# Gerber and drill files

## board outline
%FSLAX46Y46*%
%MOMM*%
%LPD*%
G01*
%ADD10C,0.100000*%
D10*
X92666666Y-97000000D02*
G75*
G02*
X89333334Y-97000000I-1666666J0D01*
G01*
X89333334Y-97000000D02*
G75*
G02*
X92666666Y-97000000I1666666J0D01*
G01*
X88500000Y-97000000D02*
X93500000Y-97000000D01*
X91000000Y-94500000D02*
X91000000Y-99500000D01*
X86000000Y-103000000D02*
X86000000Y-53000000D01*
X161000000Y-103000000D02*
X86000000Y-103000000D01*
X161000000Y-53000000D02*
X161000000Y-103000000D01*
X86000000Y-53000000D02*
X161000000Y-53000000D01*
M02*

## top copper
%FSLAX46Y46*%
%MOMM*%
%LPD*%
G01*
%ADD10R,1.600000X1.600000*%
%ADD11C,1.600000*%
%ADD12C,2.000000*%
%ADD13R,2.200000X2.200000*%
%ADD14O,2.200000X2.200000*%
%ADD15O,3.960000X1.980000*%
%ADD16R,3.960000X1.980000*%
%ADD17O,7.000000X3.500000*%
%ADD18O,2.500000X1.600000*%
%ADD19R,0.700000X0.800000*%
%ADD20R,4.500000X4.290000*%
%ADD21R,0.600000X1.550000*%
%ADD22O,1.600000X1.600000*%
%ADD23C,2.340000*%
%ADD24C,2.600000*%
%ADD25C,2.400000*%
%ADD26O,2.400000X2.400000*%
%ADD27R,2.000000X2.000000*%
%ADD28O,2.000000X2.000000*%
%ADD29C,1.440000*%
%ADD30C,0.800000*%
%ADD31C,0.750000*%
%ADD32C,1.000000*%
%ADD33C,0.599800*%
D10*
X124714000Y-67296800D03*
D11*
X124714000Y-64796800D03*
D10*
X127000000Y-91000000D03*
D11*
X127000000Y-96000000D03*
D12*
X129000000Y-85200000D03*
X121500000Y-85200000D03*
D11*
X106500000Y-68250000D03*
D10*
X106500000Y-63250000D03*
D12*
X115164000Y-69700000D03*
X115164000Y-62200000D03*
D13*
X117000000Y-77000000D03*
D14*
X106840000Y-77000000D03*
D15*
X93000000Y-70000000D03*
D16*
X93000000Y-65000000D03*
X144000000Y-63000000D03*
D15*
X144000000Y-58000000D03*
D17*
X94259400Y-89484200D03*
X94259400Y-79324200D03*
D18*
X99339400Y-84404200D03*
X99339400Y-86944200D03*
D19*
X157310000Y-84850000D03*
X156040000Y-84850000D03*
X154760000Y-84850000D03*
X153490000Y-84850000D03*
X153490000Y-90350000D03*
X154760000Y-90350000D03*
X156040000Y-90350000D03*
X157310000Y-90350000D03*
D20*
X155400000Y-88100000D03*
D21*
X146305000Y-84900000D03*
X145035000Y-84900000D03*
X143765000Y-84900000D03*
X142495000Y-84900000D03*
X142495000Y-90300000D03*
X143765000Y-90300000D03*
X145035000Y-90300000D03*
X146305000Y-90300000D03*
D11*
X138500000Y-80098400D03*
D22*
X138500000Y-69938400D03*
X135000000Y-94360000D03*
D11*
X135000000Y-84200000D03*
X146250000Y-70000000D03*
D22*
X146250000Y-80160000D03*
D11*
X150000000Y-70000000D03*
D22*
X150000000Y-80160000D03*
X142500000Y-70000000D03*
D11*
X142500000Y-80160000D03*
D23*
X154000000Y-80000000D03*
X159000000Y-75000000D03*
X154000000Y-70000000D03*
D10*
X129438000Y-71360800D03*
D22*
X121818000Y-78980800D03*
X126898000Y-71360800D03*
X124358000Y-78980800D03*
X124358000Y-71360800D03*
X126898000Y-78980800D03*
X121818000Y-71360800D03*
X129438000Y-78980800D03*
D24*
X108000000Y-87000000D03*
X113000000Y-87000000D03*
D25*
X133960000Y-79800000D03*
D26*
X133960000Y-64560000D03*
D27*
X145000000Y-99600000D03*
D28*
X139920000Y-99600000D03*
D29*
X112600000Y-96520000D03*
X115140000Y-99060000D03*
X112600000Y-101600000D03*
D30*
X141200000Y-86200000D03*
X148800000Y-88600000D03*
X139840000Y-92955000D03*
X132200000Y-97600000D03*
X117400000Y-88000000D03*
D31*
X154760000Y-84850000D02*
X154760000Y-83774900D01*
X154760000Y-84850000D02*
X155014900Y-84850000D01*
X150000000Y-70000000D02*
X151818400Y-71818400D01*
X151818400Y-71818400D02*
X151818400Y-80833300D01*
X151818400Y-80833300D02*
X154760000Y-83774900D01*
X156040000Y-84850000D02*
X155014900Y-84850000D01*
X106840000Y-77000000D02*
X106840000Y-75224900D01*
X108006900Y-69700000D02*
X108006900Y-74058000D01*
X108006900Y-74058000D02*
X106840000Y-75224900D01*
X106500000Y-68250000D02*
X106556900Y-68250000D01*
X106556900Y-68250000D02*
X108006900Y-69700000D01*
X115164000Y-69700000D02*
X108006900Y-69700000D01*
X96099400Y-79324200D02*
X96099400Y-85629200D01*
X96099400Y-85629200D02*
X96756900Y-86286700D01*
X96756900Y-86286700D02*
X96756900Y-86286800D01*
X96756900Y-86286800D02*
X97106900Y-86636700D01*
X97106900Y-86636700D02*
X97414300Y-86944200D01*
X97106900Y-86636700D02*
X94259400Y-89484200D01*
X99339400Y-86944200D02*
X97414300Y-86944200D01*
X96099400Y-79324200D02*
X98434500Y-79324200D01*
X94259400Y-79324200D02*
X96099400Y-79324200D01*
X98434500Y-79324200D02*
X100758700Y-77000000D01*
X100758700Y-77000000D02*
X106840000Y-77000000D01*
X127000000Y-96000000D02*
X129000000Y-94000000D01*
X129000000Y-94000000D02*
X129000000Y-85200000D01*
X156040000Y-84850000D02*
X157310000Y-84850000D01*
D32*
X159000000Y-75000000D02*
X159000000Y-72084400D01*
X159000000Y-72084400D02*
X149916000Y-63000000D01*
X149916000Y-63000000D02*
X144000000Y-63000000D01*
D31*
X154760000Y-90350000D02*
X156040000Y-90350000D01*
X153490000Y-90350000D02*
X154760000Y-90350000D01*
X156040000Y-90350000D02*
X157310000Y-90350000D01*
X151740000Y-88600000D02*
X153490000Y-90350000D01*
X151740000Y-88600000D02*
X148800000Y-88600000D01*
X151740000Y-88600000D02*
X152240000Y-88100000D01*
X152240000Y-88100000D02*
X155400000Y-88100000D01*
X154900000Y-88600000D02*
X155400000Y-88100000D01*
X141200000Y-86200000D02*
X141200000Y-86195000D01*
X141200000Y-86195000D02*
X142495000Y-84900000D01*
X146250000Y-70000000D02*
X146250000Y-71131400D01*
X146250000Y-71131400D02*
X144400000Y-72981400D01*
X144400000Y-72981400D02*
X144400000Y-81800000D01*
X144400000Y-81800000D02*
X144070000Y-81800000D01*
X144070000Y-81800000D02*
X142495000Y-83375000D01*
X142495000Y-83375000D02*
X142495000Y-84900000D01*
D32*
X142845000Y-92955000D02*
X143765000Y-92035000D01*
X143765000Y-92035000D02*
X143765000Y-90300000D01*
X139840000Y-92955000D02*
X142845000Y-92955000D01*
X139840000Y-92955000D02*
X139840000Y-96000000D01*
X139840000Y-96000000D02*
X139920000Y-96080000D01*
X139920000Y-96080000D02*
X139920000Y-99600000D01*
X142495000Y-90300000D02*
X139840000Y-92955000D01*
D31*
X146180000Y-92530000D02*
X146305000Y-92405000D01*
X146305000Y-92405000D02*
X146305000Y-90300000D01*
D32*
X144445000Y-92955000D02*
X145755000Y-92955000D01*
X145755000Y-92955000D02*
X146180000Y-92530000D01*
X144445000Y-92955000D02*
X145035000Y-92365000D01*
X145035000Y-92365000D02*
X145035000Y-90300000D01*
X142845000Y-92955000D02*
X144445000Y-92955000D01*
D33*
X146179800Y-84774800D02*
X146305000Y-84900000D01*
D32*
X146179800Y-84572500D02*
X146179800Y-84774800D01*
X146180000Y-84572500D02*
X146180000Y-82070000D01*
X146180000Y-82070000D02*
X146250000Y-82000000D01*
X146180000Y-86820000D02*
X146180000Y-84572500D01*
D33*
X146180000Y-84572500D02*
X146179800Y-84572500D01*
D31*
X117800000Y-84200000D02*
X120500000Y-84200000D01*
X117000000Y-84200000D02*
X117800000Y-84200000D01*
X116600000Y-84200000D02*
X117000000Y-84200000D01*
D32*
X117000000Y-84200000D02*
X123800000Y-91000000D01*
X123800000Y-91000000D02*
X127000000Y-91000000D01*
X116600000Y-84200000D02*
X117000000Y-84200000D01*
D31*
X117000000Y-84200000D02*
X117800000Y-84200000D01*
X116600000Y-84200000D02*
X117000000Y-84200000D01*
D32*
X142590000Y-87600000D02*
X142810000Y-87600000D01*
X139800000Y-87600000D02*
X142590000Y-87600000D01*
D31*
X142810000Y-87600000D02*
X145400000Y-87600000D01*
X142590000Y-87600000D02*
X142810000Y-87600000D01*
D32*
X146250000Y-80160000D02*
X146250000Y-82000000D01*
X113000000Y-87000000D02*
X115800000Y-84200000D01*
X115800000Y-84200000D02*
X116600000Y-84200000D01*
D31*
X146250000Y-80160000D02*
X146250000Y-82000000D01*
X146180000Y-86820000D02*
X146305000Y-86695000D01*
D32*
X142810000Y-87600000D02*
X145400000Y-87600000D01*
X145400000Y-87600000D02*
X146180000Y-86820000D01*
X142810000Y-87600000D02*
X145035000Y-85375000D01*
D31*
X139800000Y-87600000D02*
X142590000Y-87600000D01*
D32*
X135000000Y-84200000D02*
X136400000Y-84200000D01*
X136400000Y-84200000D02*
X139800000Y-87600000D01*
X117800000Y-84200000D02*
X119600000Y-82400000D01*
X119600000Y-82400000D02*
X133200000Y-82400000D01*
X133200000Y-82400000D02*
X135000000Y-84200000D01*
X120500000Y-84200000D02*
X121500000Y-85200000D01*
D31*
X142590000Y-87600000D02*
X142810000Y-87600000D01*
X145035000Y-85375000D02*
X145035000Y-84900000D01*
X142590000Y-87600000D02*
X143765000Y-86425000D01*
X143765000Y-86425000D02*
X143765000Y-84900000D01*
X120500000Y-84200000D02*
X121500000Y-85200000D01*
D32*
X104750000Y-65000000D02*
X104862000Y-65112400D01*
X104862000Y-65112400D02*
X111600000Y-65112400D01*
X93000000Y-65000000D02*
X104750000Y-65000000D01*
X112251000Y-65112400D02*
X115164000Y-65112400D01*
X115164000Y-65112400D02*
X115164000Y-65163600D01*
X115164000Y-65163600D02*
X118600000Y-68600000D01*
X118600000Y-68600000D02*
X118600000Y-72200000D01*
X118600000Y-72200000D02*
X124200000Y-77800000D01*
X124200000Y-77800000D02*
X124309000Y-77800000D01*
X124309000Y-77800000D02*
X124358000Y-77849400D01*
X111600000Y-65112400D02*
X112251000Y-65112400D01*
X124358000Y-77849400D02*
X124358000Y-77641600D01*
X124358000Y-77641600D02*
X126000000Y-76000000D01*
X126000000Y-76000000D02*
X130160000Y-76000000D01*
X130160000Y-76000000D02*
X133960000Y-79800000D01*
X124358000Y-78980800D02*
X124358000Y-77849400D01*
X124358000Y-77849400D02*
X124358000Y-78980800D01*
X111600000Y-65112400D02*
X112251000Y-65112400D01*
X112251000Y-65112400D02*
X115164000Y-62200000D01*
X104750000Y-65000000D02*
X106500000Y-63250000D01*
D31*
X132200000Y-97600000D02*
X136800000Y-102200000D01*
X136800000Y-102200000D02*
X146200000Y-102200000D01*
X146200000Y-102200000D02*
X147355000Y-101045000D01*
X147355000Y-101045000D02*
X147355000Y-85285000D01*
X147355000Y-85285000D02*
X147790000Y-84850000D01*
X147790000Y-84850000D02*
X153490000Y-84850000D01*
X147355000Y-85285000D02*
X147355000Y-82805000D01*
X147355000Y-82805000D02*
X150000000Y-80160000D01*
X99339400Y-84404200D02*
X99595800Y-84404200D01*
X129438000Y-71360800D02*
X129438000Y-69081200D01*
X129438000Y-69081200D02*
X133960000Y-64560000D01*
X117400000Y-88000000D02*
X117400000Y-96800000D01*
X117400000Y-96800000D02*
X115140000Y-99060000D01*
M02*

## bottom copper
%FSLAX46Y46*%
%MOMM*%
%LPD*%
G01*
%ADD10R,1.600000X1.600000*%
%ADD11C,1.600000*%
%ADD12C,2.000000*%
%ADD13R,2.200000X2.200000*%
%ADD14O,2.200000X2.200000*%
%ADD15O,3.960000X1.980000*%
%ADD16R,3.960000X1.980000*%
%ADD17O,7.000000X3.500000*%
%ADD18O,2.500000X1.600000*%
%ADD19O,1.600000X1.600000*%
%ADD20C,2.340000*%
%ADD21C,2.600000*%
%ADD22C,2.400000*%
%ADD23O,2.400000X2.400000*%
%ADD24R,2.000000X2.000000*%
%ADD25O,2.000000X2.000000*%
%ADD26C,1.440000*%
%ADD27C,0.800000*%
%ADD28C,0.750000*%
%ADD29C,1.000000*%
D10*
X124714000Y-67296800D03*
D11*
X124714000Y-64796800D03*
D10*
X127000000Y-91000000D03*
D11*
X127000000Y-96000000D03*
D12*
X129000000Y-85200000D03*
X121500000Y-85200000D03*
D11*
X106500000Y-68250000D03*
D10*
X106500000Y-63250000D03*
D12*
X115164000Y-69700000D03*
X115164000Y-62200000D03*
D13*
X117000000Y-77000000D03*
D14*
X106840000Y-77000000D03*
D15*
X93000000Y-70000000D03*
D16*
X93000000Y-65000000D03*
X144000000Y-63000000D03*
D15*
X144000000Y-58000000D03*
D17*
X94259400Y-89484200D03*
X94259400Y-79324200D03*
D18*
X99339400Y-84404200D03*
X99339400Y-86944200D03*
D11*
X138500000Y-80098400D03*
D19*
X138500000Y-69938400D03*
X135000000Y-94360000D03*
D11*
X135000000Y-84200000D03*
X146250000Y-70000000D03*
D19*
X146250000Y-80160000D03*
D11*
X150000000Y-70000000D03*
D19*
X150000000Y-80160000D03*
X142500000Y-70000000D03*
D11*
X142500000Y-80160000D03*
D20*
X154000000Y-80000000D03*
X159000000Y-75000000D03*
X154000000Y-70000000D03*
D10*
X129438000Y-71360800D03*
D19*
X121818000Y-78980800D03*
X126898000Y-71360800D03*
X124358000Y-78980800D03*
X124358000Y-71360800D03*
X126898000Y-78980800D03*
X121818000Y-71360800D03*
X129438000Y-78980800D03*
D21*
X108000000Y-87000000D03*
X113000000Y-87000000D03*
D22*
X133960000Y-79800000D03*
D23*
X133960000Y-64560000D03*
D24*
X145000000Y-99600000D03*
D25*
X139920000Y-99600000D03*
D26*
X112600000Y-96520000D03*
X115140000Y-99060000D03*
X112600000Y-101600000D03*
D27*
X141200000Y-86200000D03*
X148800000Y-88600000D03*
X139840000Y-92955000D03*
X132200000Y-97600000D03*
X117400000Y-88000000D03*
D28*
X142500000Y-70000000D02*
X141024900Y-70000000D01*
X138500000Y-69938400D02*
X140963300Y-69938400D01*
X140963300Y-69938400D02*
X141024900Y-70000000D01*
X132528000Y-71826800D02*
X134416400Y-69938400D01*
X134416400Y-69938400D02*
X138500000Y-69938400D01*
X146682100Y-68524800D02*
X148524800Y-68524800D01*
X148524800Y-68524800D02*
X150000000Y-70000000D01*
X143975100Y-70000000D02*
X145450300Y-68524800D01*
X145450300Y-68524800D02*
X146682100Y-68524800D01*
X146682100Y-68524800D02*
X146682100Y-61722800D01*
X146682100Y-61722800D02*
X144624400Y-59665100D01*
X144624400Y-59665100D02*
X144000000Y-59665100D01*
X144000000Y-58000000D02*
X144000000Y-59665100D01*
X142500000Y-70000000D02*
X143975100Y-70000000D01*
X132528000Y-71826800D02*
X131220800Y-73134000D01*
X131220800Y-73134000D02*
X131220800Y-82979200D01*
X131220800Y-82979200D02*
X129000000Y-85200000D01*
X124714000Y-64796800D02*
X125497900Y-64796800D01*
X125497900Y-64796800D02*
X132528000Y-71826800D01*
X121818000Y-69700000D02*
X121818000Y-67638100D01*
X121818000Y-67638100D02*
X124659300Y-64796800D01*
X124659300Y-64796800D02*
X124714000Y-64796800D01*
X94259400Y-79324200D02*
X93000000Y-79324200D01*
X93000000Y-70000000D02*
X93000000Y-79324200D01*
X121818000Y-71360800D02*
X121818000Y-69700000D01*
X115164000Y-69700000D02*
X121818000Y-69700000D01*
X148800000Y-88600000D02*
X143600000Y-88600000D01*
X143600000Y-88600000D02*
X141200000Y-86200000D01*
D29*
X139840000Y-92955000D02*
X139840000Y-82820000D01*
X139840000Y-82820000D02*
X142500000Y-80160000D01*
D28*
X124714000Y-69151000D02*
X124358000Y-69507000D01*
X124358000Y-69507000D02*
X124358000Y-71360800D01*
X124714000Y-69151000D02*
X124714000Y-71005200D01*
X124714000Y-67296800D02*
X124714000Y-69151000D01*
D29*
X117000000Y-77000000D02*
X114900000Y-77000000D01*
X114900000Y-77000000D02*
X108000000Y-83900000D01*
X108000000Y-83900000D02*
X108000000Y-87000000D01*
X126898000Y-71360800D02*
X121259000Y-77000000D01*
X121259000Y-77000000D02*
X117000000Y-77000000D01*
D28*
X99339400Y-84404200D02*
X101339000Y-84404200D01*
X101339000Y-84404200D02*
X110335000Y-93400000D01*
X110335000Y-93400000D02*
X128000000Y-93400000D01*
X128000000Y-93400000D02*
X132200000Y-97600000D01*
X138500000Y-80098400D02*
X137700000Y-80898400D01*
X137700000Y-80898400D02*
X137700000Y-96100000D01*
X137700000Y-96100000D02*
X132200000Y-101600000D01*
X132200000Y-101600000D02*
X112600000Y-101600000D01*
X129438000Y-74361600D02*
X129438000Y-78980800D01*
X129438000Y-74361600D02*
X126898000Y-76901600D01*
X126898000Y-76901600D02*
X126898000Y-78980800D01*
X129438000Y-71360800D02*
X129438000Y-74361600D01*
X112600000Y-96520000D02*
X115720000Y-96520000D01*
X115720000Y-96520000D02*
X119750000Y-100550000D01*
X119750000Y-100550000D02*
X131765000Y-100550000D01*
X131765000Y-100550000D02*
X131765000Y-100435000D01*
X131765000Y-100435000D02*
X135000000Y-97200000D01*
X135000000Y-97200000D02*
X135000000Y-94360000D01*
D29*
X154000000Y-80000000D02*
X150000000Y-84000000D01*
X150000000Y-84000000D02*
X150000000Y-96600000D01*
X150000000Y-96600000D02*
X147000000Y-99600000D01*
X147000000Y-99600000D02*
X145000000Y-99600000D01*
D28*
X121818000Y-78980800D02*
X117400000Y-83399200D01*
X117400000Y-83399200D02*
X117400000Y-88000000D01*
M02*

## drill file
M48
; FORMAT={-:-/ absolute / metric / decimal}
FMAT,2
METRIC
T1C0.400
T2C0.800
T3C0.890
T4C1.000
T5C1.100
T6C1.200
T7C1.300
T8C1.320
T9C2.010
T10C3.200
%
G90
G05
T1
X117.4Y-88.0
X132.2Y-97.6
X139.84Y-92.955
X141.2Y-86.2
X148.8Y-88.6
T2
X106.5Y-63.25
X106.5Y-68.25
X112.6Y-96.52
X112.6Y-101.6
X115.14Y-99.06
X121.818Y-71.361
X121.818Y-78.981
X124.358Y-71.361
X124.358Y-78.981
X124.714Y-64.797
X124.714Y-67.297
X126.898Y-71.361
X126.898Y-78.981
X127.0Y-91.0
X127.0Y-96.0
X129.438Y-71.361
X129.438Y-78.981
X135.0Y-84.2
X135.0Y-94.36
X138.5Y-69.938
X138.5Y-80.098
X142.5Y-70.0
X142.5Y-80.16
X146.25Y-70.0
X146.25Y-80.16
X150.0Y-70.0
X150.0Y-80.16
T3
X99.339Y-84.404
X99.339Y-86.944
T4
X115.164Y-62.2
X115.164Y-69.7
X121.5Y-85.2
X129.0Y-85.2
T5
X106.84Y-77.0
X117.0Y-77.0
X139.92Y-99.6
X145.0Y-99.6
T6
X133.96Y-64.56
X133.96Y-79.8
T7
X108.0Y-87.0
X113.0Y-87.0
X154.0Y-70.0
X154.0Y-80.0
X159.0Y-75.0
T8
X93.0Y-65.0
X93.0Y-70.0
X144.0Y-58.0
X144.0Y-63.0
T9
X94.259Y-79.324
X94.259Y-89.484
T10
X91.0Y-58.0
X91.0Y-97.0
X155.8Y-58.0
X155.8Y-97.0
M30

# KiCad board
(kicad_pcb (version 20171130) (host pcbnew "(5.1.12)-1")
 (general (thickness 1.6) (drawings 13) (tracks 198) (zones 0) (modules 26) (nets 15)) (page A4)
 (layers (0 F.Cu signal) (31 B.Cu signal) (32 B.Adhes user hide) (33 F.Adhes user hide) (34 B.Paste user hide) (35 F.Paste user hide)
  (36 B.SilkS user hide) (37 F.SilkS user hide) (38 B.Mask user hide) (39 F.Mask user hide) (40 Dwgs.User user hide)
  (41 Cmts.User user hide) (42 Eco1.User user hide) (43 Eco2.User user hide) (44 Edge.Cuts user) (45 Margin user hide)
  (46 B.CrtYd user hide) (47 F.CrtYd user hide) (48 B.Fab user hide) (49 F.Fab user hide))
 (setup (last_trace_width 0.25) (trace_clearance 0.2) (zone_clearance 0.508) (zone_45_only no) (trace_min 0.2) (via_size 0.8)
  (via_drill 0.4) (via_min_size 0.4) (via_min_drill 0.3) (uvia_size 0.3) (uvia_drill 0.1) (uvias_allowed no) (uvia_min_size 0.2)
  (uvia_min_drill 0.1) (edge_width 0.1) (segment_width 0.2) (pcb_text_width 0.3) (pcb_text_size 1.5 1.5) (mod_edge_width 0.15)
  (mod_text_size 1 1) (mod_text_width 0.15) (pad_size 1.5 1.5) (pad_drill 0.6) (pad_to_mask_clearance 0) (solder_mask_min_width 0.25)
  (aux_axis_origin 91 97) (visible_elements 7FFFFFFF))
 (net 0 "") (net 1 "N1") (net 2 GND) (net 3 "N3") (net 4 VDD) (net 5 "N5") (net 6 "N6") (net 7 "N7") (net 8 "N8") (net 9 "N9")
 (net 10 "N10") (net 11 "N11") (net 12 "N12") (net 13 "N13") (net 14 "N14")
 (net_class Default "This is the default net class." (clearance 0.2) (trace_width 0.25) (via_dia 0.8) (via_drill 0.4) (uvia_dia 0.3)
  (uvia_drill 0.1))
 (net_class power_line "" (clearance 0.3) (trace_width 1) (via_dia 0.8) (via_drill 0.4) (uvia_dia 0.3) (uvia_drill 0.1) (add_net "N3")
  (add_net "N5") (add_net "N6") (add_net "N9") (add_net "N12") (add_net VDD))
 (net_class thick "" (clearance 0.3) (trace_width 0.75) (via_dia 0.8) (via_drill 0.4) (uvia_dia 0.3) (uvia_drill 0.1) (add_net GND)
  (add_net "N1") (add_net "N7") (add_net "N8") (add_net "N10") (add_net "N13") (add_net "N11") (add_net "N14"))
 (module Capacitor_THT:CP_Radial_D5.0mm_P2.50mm (layer F.Cu) (at 124.714 67.2968 90)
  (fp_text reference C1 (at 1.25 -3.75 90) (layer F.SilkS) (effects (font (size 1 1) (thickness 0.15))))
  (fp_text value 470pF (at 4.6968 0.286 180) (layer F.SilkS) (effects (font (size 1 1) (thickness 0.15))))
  (pad 1 thru_hole rect (at 0 0 90) (size 1.6 1.6) (drill 0.8) (layers *.Cu *.Mask) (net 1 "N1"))
  (pad 2 thru_hole circle (at 2.5 0 90) (size 1.6 1.6) (drill 0.8) (layers *.Cu *.Mask) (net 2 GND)))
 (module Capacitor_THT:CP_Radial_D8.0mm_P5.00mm (layer F.Cu) (at 127 91 270)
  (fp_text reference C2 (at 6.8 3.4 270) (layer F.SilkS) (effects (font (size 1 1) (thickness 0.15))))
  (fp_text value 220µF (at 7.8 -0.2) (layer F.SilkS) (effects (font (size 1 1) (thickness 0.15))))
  (pad 1 thru_hole rect (at 0 0 270) (size 1.6 1.6) (drill 0.8) (layers *.Cu *.Mask) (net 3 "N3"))
  (pad 2 thru_hole circle (at 5 0 270) (size 1.6 1.6) (drill 0.8) (layers *.Cu *.Mask) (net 2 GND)))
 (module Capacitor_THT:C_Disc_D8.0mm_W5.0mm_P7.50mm (layer F.Cu) (at 129 85.2 180)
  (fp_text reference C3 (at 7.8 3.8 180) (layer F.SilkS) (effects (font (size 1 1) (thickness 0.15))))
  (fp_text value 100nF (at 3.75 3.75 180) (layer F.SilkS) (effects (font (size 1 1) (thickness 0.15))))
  (pad 1 thru_hole circle (at 0 0 180) (size 2 2) (drill 1) (layers *.Cu *.Mask) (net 2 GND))
  (pad 2 thru_hole circle (at 7.5 0 180) (size 2 2) (drill 1) (layers *.Cu *.Mask) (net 3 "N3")))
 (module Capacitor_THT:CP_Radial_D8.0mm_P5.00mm (layer F.Cu) (at 106.5 63.25 270)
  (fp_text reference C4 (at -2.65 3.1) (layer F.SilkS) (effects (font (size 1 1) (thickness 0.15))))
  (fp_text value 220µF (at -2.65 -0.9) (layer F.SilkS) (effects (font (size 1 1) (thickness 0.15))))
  (pad 2 thru_hole circle (at 5 0 270) (size 1.6 1.6) (drill 0.8) (layers *.Cu *.Mask) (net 2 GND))
  (pad 1 thru_hole rect (at 0 0 270) (size 1.6 1.6) (drill 0.8) (layers *.Cu *.Mask) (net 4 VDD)))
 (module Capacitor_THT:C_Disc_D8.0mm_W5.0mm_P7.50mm (layer F.Cu) (at 115.164 62.2 270)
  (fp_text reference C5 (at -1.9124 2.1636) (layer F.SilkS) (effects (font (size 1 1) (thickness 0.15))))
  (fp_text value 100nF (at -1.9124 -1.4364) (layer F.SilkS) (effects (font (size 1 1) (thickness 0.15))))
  (pad 2 thru_hole circle (at 7.5 0 270) (size 2 2) (drill 1) (layers *.Cu *.Mask) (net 2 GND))
  (pad 1 thru_hole circle (at 0 0 270) (size 2 2) (drill 1) (layers *.Cu *.Mask) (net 4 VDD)))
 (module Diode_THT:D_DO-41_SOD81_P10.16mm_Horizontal (layer F.Cu) (at 117 77 180)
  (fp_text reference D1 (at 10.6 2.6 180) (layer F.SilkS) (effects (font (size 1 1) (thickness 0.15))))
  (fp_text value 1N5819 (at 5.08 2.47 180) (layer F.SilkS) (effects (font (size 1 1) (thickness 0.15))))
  (pad 1 thru_hole rect (at 0 0 180) (size 2.2 2.2) (drill 1.1) (layers *.Cu *.Mask) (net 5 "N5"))
  (pad 2 thru_hole oval (at 10.16 0 180) (size 2.2 2.2) (drill 1.1) (layers *.Cu *.Mask) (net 2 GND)))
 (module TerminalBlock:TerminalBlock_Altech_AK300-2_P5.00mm (layer F.Cu) (at 93 65 270)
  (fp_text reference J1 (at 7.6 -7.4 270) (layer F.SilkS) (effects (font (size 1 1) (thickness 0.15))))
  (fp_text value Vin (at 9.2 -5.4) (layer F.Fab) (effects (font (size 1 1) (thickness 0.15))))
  (pad 2 thru_hole oval (at 5 0 270) (size 1.98 3.96) (drill 1.32) (layers *.Cu *.Mask) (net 2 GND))
  (pad 1 thru_hole rect (at 0 0 270) (size 1.98 3.96) (drill 1.32) (layers *.Cu *.Mask) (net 4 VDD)))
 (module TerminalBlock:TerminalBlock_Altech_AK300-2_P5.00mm (layer F.Cu) (at 144 63 90)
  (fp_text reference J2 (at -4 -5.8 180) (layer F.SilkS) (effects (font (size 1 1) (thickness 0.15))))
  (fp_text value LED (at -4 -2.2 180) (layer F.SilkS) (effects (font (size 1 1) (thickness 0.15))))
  (pad 1 thru_hole rect (at 0 0 90) (size 1.98 3.96) (drill 1.32) (layers *.Cu *.Mask) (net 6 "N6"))
  (pad 2 thru_hole oval (at 5 0 90) (size 1.98 3.96) (drill 1.32) (layers *.Cu *.Mask) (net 2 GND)))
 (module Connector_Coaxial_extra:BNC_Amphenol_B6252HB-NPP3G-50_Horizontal (layer F.Cu) (at 99.3394 84.4042 90)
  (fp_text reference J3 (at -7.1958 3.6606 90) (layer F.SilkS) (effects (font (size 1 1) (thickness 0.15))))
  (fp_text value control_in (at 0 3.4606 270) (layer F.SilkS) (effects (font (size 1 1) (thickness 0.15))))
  (pad 2 thru_hole oval (at -5.08 -5.08 90) (size 3.5 7) (drill 2.01) (layers *.Cu *.Mask) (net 2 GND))
  (pad 2 thru_hole oval (at 5.08 -5.08 90) (size 3.5 7) (drill 2.01) (layers *.Cu *.Mask) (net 2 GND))
  (pad 1 thru_hole oval (at 0 0 90) (size 1.6 2.5) (drill 0.89) (layers *.Cu *.Mask) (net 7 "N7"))
  (pad 2 thru_hole oval (at -2.54 0 90) (size 1.6 2.5) (drill 0.89) (layers *.Cu *.Mask) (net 2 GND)))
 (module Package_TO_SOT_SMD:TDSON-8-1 (layer F.Cu) (at 155.4 87.6 270)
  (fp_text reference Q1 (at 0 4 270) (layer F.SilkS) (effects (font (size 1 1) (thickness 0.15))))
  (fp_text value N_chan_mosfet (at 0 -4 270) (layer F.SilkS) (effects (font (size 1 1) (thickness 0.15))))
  (pad 1 smd rect (at -2.75 -1.91 180) (size 0.7 0.8) (layers F.Cu F.Paste F.Mask) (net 2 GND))
  (pad 2 smd rect (at -2.75 -0.64 180) (size 0.7 0.8) (layers F.Cu F.Paste F.Mask) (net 2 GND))
  (pad 3 smd rect (at -2.75 0.64 180) (size 0.7 0.8) (layers F.Cu F.Paste F.Mask) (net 2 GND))
  (pad 4 smd rect (at -2.75 1.91 180) (size 0.7 0.8) (layers F.Cu F.Paste F.Mask) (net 7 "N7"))
  (pad 5 smd rect (at 2.75 1.91 180) (size 0.7 0.8) (layers F.Cu F.Paste F.Mask) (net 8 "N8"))
  (pad 5 smd rect (at 2.75 0.64 180) (size 0.7 0.8) (layers F.Cu F.Paste F.Mask) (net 8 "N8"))
  (pad 5 smd rect (at 2.75 -0.64 180) (size 0.7 0.8) (layers F.Cu F.Paste F.Mask) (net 8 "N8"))
  (pad 5 smd rect (at 2.75 -1.91 180) (size 0.7 0.8) (layers F.Cu F.Paste F.Mask) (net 8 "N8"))
  (pad 5 smd rect (at 0.5 0 180) (size 4.5 4.29) (layers F.Cu F.Mask) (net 8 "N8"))
  (pad "" smd rect (at 1.25 -1.09 180) (size 1.55 1.6) (layers F.Paste))
  (pad "" smd rect (at 1.25 1.09 180) (size 1.55 1.6) (layers F.Paste))
  (pad "" smd rect (at -0.75 -1.09 180) (size 1.55 1.2) (layers F.Paste))
  (pad "" smd rect (at -0.75 1.09 180) (size 1.55 1.2) (layers F.Paste)))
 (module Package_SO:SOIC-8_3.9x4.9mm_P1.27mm (layer F.Cu) (at 144.4 87.6 270)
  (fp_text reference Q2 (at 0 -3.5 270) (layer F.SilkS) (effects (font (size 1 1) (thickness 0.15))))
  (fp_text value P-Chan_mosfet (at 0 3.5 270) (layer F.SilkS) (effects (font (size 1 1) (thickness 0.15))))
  (pad 1 smd rect (at -2.7 -1.905 270) (size 1.55 0.6) (layers F.Cu F.Paste F.Mask) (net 3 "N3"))
  (pad 2 smd rect (at -2.7 -0.635 270) (size 1.55 0.6) (layers F.Cu F.Paste F.Mask) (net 3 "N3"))
  (pad 3 smd rect (at -2.7 0.635 270) (size 1.55 0.6) (layers F.Cu F.Paste F.Mask) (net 3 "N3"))
  (pad 4 smd rect (at -2.7 1.905 270) (size 1.55 0.6) (layers F.Cu F.Paste F.Mask) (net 8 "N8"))
  (pad 5 smd rect (at 2.7 1.905 270) (size 1.55 0.6) (layers F.Cu F.Paste F.Mask) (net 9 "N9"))
  (pad 6 smd rect (at 2.7 0.635 270) (size 1.55 0.6) (layers F.Cu F.Paste F.Mask) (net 9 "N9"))
  (pad 7 smd rect (at 2.7 -0.635 270) (size 1.55 0.6) (layers F.Cu F.Paste F.Mask) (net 9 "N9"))
  (pad 8 smd rect (at 2.7 -1.905 270) (size 1.55 0.6) (layers F.Cu F.Paste F.Mask) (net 9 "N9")))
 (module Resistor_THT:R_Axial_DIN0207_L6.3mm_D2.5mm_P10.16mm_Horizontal (layer F.Cu) (at 138.5 80.0984 90)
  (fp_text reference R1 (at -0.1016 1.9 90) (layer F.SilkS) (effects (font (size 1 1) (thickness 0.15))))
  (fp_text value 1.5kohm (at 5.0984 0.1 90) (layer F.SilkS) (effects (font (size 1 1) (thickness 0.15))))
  (pad 1 thru_hole circle (at 0 0 90) (size 1.6 1.6) (drill 0.8) (layers *.Cu *.Mask) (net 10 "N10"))
  (pad 2 thru_hole oval (at 10.16 0 90) (size 1.6 1.6) (drill 0.8) (layers *.Cu *.Mask) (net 2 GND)))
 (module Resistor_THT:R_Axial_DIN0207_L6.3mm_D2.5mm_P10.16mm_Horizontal (layer F.Cu) (at 135 84.2 270)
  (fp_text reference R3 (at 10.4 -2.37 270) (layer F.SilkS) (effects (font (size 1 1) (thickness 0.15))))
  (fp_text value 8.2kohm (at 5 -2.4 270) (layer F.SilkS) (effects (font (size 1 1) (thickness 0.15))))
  (pad 2 thru_hole oval (at 10.16 0 270) (size 1.6 1.6) (drill 0.8) (layers *.Cu *.Mask) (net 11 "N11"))
  (pad 1 thru_hole circle (at 0 0 270) (size 1.6 1.6) (drill 0.8) (layers *.Cu *.Mask) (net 3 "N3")))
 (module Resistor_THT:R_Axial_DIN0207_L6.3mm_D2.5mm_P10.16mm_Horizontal (layer F.Cu) (at 146.25 70 270)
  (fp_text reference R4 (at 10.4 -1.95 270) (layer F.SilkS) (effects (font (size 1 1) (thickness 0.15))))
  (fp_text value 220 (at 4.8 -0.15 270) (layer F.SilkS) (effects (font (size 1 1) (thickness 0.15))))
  (pad 1 thru_hole circle (at 0 0 270) (size 1.6 1.6) (drill 0.8) (layers *.Cu *.Mask) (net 8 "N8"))
  (pad 2 thru_hole oval (at 10.16 0 270) (size 1.6 1.6) (drill 0.8) (layers *.Cu *.Mask) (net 3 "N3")))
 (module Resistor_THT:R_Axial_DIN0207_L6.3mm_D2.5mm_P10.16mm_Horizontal (layer F.Cu) (at 150 70 270)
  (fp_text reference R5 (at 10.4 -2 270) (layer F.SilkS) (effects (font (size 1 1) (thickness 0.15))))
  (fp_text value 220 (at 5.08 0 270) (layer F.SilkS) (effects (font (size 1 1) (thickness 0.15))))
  (pad 1 thru_hole circle (at 0 0 270) (size 1.6 1.6) (drill 0.8) (layers *.Cu *.Mask) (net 2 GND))
  (pad 2 thru_hole oval (at 10.16 0 270) (size 1.6 1.6) (drill 0.8) (layers *.Cu *.Mask) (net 7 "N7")))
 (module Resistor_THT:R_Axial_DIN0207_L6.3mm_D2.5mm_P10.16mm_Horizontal (layer F.Cu) (at 142.5 80.16 90)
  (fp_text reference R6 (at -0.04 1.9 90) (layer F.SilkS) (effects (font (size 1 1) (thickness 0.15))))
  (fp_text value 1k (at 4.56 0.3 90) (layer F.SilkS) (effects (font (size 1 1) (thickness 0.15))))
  (pad 2 thru_hole oval (at 10.16 0 90) (size 1.6 1.6) (drill 0.8) (layers *.Cu *.Mask) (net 2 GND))
  (pad 1 thru_hole circle (at 0 0 90) (size 1.6 1.6) (drill 0.8) (layers *.Cu *.Mask) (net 9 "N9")))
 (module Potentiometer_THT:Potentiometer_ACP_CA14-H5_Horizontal (layer F.Cu) (at 154 70)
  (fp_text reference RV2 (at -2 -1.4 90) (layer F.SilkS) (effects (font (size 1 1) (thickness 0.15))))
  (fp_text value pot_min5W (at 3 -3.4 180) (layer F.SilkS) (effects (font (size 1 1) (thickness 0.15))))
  (pad 3 thru_hole circle (at 0 10) (size 2.34 2.34) (drill 1.3) (layers *.Cu *.Mask) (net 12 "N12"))
  (pad 2 thru_hole circle (at 5 5) (size 2.34 2.34) (drill 1.3) (layers *.Cu *.Mask) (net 6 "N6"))
  (pad 1 thru_hole circle (at 0 0) (size 2.34 2.34) (drill 1.3) (layers *.Cu *.Mask)))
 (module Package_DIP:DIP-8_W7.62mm (layer F.Cu) (at 129.438 71.3608 270)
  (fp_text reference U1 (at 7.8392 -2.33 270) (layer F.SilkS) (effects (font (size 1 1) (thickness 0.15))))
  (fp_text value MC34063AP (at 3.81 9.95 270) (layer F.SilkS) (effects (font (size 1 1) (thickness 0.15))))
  (pad 1 thru_hole rect (at 0 0 270) (size 1.6 1.6) (drill 0.8) (layers *.Cu *.Mask) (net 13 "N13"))
  (pad 5 thru_hole oval (at 7.62 7.62 270) (size 1.6 1.6) (drill 0.8) (layers *.Cu *.Mask) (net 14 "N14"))
  (pad 2 thru_hole oval (at 0 2.54 270) (size 1.6 1.6) (drill 0.8) (layers *.Cu *.Mask) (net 5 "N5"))
  (pad 6 thru_hole oval (at 7.62 5.08 270) (size 1.6 1.6) (drill 0.8) (layers *.Cu *.Mask) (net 4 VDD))
  (pad 3 thru_hole oval (at 0 5.08 270) (size 1.6 1.6) (drill 0.8) (layers *.Cu *.Mask) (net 1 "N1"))
  (pad 7 thru_hole oval (at 7.62 2.54 270) (size 1.6 1.6) (drill 0.8) (layers *.Cu *.Mask) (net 13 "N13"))
  (pad 4 thru_hole oval (at 0 7.62 270) (size 1.6 1.6) (drill 0.8) (layers *.Cu *.Mask) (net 2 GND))
  (pad 8 thru_hole oval (at 7.62 0 270) (size 1.6 1.6) (drill 0.8) (layers *.Cu *.Mask) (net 13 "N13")))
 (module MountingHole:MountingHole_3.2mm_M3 (layer F.Cu) (at 91 58)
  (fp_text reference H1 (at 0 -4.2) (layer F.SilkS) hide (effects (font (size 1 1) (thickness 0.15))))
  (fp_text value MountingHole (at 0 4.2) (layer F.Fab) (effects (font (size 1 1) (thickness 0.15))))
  (pad 1 np_thru_hole circle (at 0 0) (size 3.2 3.2) (drill 3.2) (layers *.Cu *.Mask)))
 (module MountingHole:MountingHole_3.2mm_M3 (layer F.Cu) (at 155.8 97)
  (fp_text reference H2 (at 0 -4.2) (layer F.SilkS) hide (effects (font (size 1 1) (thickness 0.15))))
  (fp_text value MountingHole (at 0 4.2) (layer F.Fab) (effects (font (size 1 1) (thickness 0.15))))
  (pad 1 np_thru_hole circle (at 0 0) (size 3.2 3.2) (drill 3.2) (layers *.Cu *.Mask)))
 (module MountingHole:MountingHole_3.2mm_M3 (layer F.Cu) (at 91 97)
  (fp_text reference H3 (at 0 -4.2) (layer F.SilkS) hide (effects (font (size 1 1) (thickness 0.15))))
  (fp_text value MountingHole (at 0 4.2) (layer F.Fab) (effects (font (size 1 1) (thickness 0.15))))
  (pad 1 np_thru_hole circle (at 0 0) (size 3.2 3.2) (drill 3.2) (layers *.Cu *.Mask)))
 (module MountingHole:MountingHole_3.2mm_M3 (layer F.Cu) (at 155.8 58)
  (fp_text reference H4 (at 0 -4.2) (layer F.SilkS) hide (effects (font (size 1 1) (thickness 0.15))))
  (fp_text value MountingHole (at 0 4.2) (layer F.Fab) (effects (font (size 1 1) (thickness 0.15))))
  (pad 1 np_thru_hole circle (at 0 0) (size 3.2 3.2) (drill 3.2) (layers *.Cu *.Mask)))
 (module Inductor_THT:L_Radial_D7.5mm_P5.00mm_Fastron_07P (layer F.Cu) (at 108 87)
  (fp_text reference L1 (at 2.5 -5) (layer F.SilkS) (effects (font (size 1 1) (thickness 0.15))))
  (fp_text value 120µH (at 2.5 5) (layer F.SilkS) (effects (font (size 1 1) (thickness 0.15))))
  (pad 1 thru_hole circle (at 0 0) (size 2.6 2.6) (drill 1.3) (layers *.Cu *.Mask) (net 5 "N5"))
  (pad 2 thru_hole circle (at 5 0) (size 2.6 2.6) (drill 1.3) (layers *.Cu *.Mask) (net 3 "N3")))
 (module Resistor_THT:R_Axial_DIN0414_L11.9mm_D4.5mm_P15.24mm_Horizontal (layer F.Cu) (at 133.96 79.8 90)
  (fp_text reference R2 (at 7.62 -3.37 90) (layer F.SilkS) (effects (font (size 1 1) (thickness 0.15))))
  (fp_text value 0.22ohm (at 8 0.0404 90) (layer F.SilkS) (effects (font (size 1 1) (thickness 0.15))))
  (pad 1 thru_hole circle (at 0 0 90) (size 2.4 2.4) (drill 1.2) (layers *.Cu *.Mask) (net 4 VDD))
  (pad 2 thru_hole oval (at 15.24 0 90) (size 2.4 2.4) (drill 1.2) (layers *.Cu *.Mask) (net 13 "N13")))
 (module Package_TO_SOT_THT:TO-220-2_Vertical (layer F.Cu) (at 145 99.6 180)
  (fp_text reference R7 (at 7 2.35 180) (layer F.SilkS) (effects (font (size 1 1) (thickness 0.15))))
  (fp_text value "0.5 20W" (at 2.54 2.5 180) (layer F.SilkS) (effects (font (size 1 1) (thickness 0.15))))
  (pad 1 thru_hole rect (at 0 0 180) (size 2 2) (drill 1.1) (layers *.Cu *.Mask) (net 12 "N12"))
  (pad 2 thru_hole oval (at 5.08 0 180) (size 2 2) (drill 1.1) (layers *.Cu *.Mask) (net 9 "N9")))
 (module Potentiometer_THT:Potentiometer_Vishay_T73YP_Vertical (layer F.Cu) (at 112.6 101.6)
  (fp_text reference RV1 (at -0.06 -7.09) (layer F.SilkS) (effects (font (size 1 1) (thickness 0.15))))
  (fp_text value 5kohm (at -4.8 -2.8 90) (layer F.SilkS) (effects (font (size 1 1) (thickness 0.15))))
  (pad 3 thru_hole circle (at 0 -5.08) (size 1.44 1.44) (drill 0.8) (layers *.Cu *.Mask) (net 11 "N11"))
  (pad 2 thru_hole circle (at 2.54 -2.54) (size 1.44 1.44) (drill 0.8) (layers *.Cu *.Mask) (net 14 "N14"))
  (pad 1 thru_hole circle (at 0 0) (size 1.44 1.44) (drill 0.8) (layers *.Cu *.Mask) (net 10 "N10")))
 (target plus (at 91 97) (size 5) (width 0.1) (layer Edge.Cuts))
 (gr_line (start 86 103) (end 86 53) (layer Edge.Cuts) (width 0.1))
 (gr_line (start 161 103) (end 86 103) (layer Edge.Cuts) (width 0.1))
 (gr_line (start 161 53) (end 161 103) (layer Edge.Cuts) (width 0.1))
 (gr_line (start 86 53) (end 161 53) (layer Edge.Cuts) (width 0.1))
 (segment (start 154.76 84.85) (end 154.76 83.7749) (width 0.75) (layer F.Cu) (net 2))
 (segment (start 154.76 84.85) (end 155.0149 84.85) (width 0.75) (layer F.Cu) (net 2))
 (segment (start 150 70) (end 151.8184 71.8184) (width 0.75) (layer F.Cu) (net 2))
 (segment (start 151.8184 71.8184) (end 151.8184 80.8333) (width 0.75) (layer F.Cu) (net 2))
 (segment (start 151.8184 80.8333) (end 154.76 83.7749) (width 0.75) (layer F.Cu) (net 2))
 (segment (start 156.04 84.85) (end 155.0149 84.85) (width 0.75) (layer F.Cu) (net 2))
 (segment (start 142.5 70) (end 141.0249 70) (width 0.75) (layer B.Cu) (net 2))
 (segment (start 138.5 69.9384) (end 140.9633 69.9384) (width 0.75) (layer B.Cu) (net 2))
 (segment (start 140.9633 69.9384) (end 141.0249 70) (width 0.75) (layer B.Cu) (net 2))
 (segment (start 132.528 71.8268) (end 134.4164 69.9384) (width 0.75) (layer B.Cu) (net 2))
 (segment (start 134.4164 69.9384) (end 138.5 69.9384) (width 0.75) (layer B.Cu) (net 2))
 (segment (start 106.84 77) (end 106.84 75.2249) (width 0.75) (layer F.Cu) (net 2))
 (segment (start 108.0069 69.7) (end 108.0069 74.058) (width 0.75) (layer F.Cu) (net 2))
 (segment (start 108.0069 74.058) (end 106.84 75.2249) (width 0.75) (layer F.Cu) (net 2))
 (segment (start 106.5 68.25) (end 106.5569 68.25) (width 0.75) (layer F.Cu) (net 2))
 (segment (start 106.5569 68.25) (end 108.0069 69.7) (width 0.75) (layer F.Cu) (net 2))
 (segment (start 115.164 69.7) (end 108.0069 69.7) (width 0.75) (layer F.Cu) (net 2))
 (segment (start 96.0994 79.3242) (end 96.0994 85.6292) (width 0.75) (layer F.Cu) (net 2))
 (segment (start 96.0994 85.6292) (end 96.7569 86.2867) (width 0.75) (layer F.Cu) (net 2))
 (segment (start 96.7569 86.2867) (end 96.7569 86.2868) (width 0.75) (layer F.Cu) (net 2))
 (segment (start 96.7569 86.2868) (end 97.1069 86.6367) (width 0.75) (layer F.Cu) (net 2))
 (segment (start 97.1069 86.6367) (end 97.4143 86.9442) (width 0.75) (layer F.Cu) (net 2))
 (segment (start 97.1069 86.6367) (end 94.2594 89.4842) (width 0.75) (layer F.Cu) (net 2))
 (segment (start 99.3394 86.9442) (end 97.4143 86.9442) (width 0.75) (layer F.Cu) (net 2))
 (segment (start 96.0994 79.3242) (end 98.4345 79.3242) (width 0.75) (layer F.Cu) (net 2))
 (segment (start 94.2594 79.3242) (end 96.0994 79.3242) (width 0.75) (layer F.Cu) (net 2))
 (segment (start 146.6821 68.5248) (end 148.5248 68.5248) (width 0.75) (layer B.Cu) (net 2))
 (segment (start 148.5248 68.5248) (end 150 70) (width 0.75) (layer B.Cu) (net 2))
 (segment (start 143.9751 70) (end 145.4503 68.5248) (width 0.75) (layer B.Cu) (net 2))
 (segment (start 145.4503 68.5248) (end 146.6821 68.5248) (width 0.75) (layer B.Cu) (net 2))
 (segment (start 146.6821 68.5248) (end 146.6821 61.7228) (width 0.75) (layer B.Cu) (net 2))
 (segment (start 146.6821 61.7228) (end 144.6244 59.6651) (width 0.75) (layer B.Cu) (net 2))
 (segment (start 144.6244 59.6651) (end 144 59.6651) (width 0.75) (layer B.Cu) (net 2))
 (segment (start 144 58) (end 144 59.6651) (width 0.75) (layer B.Cu) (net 2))
 (segment (start 142.5 70) (end 143.9751 70) (width 0.75) (layer B.Cu) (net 2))
 (segment (start 132.528 71.8268) (end 131.2208 73.134) (width 0.75) (layer B.Cu) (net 2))
 (segment (start 131.2208 73.134) (end 131.2208 82.9792) (width 0.75) (layer B.Cu) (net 2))
 (segment (start 131.2208 82.9792) (end 129 85.2) (width 0.75) (layer B.Cu) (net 2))
 (segment (start 124.714 64.7968) (end 125.4979 64.7968) (width 0.75) (layer B.Cu) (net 2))
 (segment (start 125.4979 64.7968) (end 132.528 71.8268) (width 0.75) (layer B.Cu) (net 2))
 (segment (start 121.818 69.7) (end 121.818 67.6381) (width 0.75) (layer B.Cu) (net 2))
 (segment (start 121.818 67.6381) (end 124.6593 64.7968) (width 0.75) (layer B.Cu) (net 2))
 (segment (start 124.6593 64.7968) (end 124.714 64.7968) (width 0.75) (layer B.Cu) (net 2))
 (segment (start 98.4345 79.3242) (end 100.7587 77) (width 0.75) (layer F.Cu) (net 2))
 (segment (start 100.7587 77) (end 106.84 77) (width 0.75) (layer F.Cu) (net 2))
 (segment (start 94.2594 79.3242) (end 93 79.3242) (width 0.75) (layer B.Cu) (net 2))
 (segment (start 93 70) (end 93 79.3242) (width 0.75) (layer B.Cu) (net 2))
 (segment (start 127 96) (end 129 94) (width 0.75) (layer F.Cu) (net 2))
 (segment (start 129 94) (end 129 85.2) (width 0.75) (layer F.Cu) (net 2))
 (segment (start 121.818 71.3608) (end 121.818 69.7) (width 0.75) (layer B.Cu) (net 2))
 (segment (start 115.164 69.7) (end 121.818 69.7) (width 0.75) (layer B.Cu) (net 2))
 (segment (start 156.04 84.85) (end 157.31 84.85) (width 0.75) (layer F.Cu) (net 2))
 (segment (start 159 75) (end 159 72.0844) (width 1) (layer F.Cu) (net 6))
 (segment (start 159 72.0844) (end 149.916 63) (width 1) (layer F.Cu) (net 6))
 (segment (start 149.916 63) (end 144 63) (width 1) (layer F.Cu) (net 6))
 (segment (start 154.76 90.35) (end 156.04 90.35) (width 0.75) (layer F.Cu) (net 8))
 (segment (start 153.49 90.35) (end 154.76 90.35) (width 0.75) (layer F.Cu) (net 8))
 (segment (start 156.04 90.35) (end 157.31 90.35) (width 0.75) (layer F.Cu) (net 8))
 (segment (start 151.74 88.6) (end 153.49 90.35) (width 0.75) (layer F.Cu) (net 8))
 (segment (start 148.8 88.6) (end 143.6 88.6) (width 0.75) (layer B.Cu) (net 8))
 (segment (start 143.6 88.6) (end 141.2 86.2) (width 0.75) (layer B.Cu) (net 8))
 (segment (start 151.74 88.6) (end 148.8 88.6) (width 0.75) (layer F.Cu) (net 8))
 (segment (start 151.74 88.6) (end 152.24 88.1) (width 0.75) (layer F.Cu) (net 8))
 (segment (start 152.24 88.1) (end 155.4 88.1) (width 0.75) (layer F.Cu) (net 8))
 (segment (start 154.9 88.6) (end 155.4 88.1) (width 0.75) (layer F.Cu) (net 8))
 (segment (start 141.2 86.2) (end 141.2 86.195) (width 0.75) (layer F.Cu) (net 8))
 (segment (start 141.2 86.195) (end 142.495 84.9) (width 0.75) (layer F.Cu) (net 8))
 (segment (start 146.25 70) (end 146.25 71.1314) (width 0.75) (layer F.Cu) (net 8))
 (segment (start 146.25 71.1314) (end 144.4 72.9814) (width 0.75) (layer F.Cu) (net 8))
 (segment (start 144.4 72.9814) (end 144.4 81.8) (width 0.75) (layer F.Cu) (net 8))
 (segment (start 144.4 81.8) (end 144.07 81.8) (width 0.75) (layer F.Cu) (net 8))
 (segment (start 144.07 81.8) (end 142.495 83.375) (width 0.75) (layer F.Cu) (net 8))
 (segment (start 142.495 83.375) (end 142.495 84.9) (width 0.75) (layer F.Cu) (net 8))
 (via (at 141.2 86.2) (size 0.8) (layers F.Cu B.Cu) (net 8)) (via (at 148.8 88.6) (size 0.8) (layers F.Cu B.Cu) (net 8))
 (segment (start 142.845 92.955) (end 143.765 92.035) (width 1) (layer F.Cu) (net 9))
 (segment (start 143.765 92.035) (end 143.765 90.3) (width 1) (layer F.Cu) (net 9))
 (segment (start 139.84 92.955) (end 142.845 92.955) (width 1) (layer F.Cu) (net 9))
 (segment (start 139.84 92.955) (end 139.84 96) (width 1) (layer F.Cu) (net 9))
 (segment (start 139.84 96) (end 139.92 96.08) (width 1) (layer F.Cu) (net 9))
 (segment (start 139.92 96.08) (end 139.92 99.6) (width 1) (layer F.Cu) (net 9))
 (segment (start 142.495 90.3) (end 139.84 92.955) (width 1) (layer F.Cu) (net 9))
 (segment (start 139.84 92.955) (end 139.84 82.82) (width 1) (layer B.Cu) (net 9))
 (segment (start 139.84 82.82) (end 142.5 80.16) (width 1) (layer B.Cu) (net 9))
 (segment (start 146.18 92.53) (end 146.305 92.405) (width 0.75) (layer F.Cu) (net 9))
 (segment (start 146.305 92.405) (end 146.305 90.3) (width 0.75) (layer F.Cu) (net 9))
 (segment (start 144.445 92.955) (end 145.755 92.955) (width 1) (layer F.Cu) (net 9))
 (segment (start 145.755 92.955) (end 146.18 92.53) (width 1) (layer F.Cu) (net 9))
 (segment (start 144.445 92.955) (end 145.035 92.365) (width 1) (layer F.Cu) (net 9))
 (segment (start 145.035 92.365) (end 145.035 90.3) (width 1) (layer F.Cu) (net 9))
 (segment (start 142.845 92.955) (end 144.445 92.955) (width 1) (layer F.Cu) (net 9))
 (via (at 139.84 92.955) (size 0.8) (layers F.Cu B.Cu) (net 9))
 (segment (start 124.714 69.151) (end 124.358 69.507) (width 0.75) (layer B.Cu) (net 1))
 (segment (start 124.358 69.507) (end 124.358 71.3608) (width 0.75) (layer B.Cu) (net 1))
 (segment (start 124.714 69.151) (end 124.714 71.0052) (width 0.75) (layer B.Cu) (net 1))
 (segment (start 124.714 67.2968) (end 124.714 69.151) (width 0.75) (layer B.Cu) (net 1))
 (segment (start 146.1798 84.7748) (end 146.305 84.9) (width 0.5998) (layer F.Cu) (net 3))
 (segment (start 146.1798 84.5725) (end 146.1798 84.7748) (width 1) (layer F.Cu) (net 3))
 (segment (start 146.18 84.5725) (end 146.18 82.07) (width 1) (layer F.Cu) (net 3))
 (segment (start 146.18 82.07) (end 146.25 82) (width 1) (layer F.Cu) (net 3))
 (segment (start 146.18 86.82) (end 146.18 84.5725) (width 1) (layer F.Cu) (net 3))
 (segment (start 146.18 84.5725) (end 146.1798 84.5725) (width 0.5998) (layer F.Cu) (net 3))
 (segment (start 117.8 84.2) (end 120.5 84.2) (width 0.75) (layer F.Cu) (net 3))
 (segment (start 117 84.2) (end 117.8 84.2) (width 0.75) (layer F.Cu) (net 3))
 (segment (start 116.6 84.2) (end 117 84.2) (width 0.75) (layer F.Cu) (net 3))
 (segment (start 117 84.2) (end 123.8 91) (width 1) (layer F.Cu) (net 3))
 (segment (start 123.8 91) (end 127 91) (width 1) (layer F.Cu) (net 3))
 (segment (start 116.6 84.2) (end 117 84.2) (width 1) (layer F.Cu) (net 3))
 (segment (start 117 84.2) (end 117.8 84.2) (width 0.75) (layer F.Cu) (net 3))
 (segment (start 116.6 84.2) (end 117 84.2) (width 0.75) (layer F.Cu) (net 3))
 (segment (start 142.59 87.6) (end 142.81 87.6) (width 1) (layer F.Cu) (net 3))
 (segment (start 139.8 87.6) (end 142.59 87.6) (width 1) (layer F.Cu) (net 3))
 (segment (start 142.81 87.6) (end 145.4 87.6) (width 0.75) (layer F.Cu) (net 3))
 (segment (start 142.59 87.6) (end 142.81 87.6) (width 0.75) (layer F.Cu) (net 3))
 (segment (start 146.25 80.16) (end 146.25 82) (width 1) (layer F.Cu) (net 3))
 (segment (start 113 87) (end 115.8 84.2) (width 1) (layer F.Cu) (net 3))
 (segment (start 115.8 84.2) (end 116.6 84.2) (width 1) (layer F.Cu) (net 3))
 (segment (start 146.25 80.16) (end 146.25 82) (width 0.75) (layer F.Cu) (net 3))
 (segment (start 146.18 86.82) (end 146.305 86.695) (width 0.75) (layer F.Cu) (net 3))
 (segment (start 142.81 87.6) (end 145.4 87.6) (width 1) (layer F.Cu) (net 3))
 (segment (start 145.4 87.6) (end 146.18 86.82) (width 1) (layer F.Cu) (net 3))
 (segment (start 142.81 87.6) (end 145.035 85.375) (width 1) (layer F.Cu) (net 3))
 (segment (start 139.8 87.6) (end 142.59 87.6) (width 0.75) (layer F.Cu) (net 3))
 (segment (start 135 84.2) (end 136.4 84.2) (width 1) (layer F.Cu) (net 3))
 (segment (start 136.4 84.2) (end 139.8 87.6) (width 1) (layer F.Cu) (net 3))
 (segment (start 117.8 84.2) (end 119.6 82.4) (width 1) (layer F.Cu) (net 3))
 (segment (start 119.6 82.4) (end 133.2 82.4) (width 1) (layer F.Cu) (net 3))
 (segment (start 133.2 82.4) (end 135 84.2) (width 1) (layer F.Cu) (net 3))
 (segment (start 120.5 84.2) (end 121.5 85.2) (width 1) (layer F.Cu) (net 3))
 (segment (start 142.59 87.6) (end 142.81 87.6) (width 0.75) (layer F.Cu) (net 3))
 (segment (start 145.035 85.375) (end 145.035 84.9) (width 0.75) (layer F.Cu) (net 3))
 (segment (start 142.59 87.6) (end 143.765 86.425) (width 0.75) (layer F.Cu) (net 3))
 (segment (start 143.765 86.425) (end 143.765 84.9) (width 0.75) (layer F.Cu) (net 3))
 (segment (start 120.5 84.2) (end 121.5 85.2) (width 0.75) (layer F.Cu) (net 3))
 (segment (start 104.75 65) (end 104.862 65.1124) (width 1) (layer F.Cu) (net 4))
 (segment (start 104.862 65.1124) (end 111.6 65.1124) (width 1) (layer F.Cu) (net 4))
 (segment (start 93 65) (end 104.75 65) (width 1) (layer F.Cu) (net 4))
 (segment (start 112.251 65.1124) (end 115.164 65.1124) (width 1) (layer F.Cu) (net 4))
 (segment (start 115.164 65.1124) (end 115.164 65.1636) (width 1) (layer F.Cu) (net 4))
 (segment (start 115.164 65.1636) (end 118.6 68.6) (width 1) (layer F.Cu) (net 4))
 (segment (start 118.6 68.6) (end 118.6 72.2) (width 1) (layer F.Cu) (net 4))
 (segment (start 118.6 72.2) (end 124.2 77.8) (width 1) (layer F.Cu) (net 4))
 (segment (start 124.2 77.8) (end 124.309 77.8) (width 1) (layer F.Cu) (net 4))
 (segment (start 124.309 77.8) (end 124.358 77.8494) (width 1) (layer F.Cu) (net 4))
 (segment (start 111.6 65.1124) (end 112.251 65.1124) (width 1) (layer F.Cu) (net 4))
 (segment (start 124.358 77.8494) (end 124.358 77.6416) (width 1) (layer F.Cu) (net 4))
 (segment (start 124.358 77.6416) (end 126 76) (width 1) (layer F.Cu) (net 4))
 (segment (start 126 76) (end 130.16 76) (width 1) (layer F.Cu) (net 4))
 (segment (start 130.16 76) (end 133.96 79.8) (width 1) (layer F.Cu) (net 4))
 (segment (start 124.358 78.9808) (end 124.358 77.8494) (width 1) (layer F.Cu) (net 4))
 (segment (start 124.358 77.8494) (end 124.358 78.9808) (width 1) (layer F.Cu) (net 4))
 (segment (start 111.6 65.1124) (end 112.251 65.1124) (width 1) (layer F.Cu) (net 4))
 (segment (start 112.251 65.1124) (end 115.164 62.2) (width 1) (layer F.Cu) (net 4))
 (segment (start 104.75 65) (end 106.5 63.25) (width 1) (layer F.Cu) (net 4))
 (segment (start 117 77) (end 114.9 77) (width 1) (layer B.Cu) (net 5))
 (segment (start 114.9 77) (end 108 83.9) (width 1) (layer B.Cu) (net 5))
 (segment (start 108 83.9) (end 108 87) (width 1) (layer B.Cu) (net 5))
 (segment (start 126.898 71.3608) (end 121.259 77) (width 1) (layer B.Cu) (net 5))
 (segment (start 121.259 77) (end 117 77) (width 1) (layer B.Cu) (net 5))
 (segment (start 132.2 97.6) (end 136.8 102.2) (width 0.75) (layer F.Cu) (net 7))
 (segment (start 136.8 102.2) (end 146.2 102.2) (width 0.75) (layer F.Cu) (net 7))
 (segment (start 146.2 102.2) (end 147.355 101.045) (width 0.75) (layer F.Cu) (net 7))
 (segment (start 147.355 101.045) (end 147.355 85.285) (width 0.75) (layer F.Cu) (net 7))
 (segment (start 99.3394 84.4042) (end 101.339 84.4042) (width 0.75) (layer B.Cu) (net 7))
 (segment (start 101.339 84.4042) (end 110.335 93.4) (width 0.75) (layer B.Cu) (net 7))
 (segment (start 110.335 93.4) (end 128 93.4) (width 0.75) (layer B.Cu) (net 7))
 (segment (start 128 93.4) (end 132.2 97.6) (width 0.75) (layer B.Cu) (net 7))
 (segment (start 147.355 85.285) (end 147.79 84.85) (width 0.75) (layer F.Cu) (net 7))
 (segment (start 147.79 84.85) (end 153.49 84.85) (width 0.75) (layer F.Cu) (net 7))
 (segment (start 147.355 85.285) (end 147.355 82.805) (width 0.75) (layer F.Cu) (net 7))
 (segment (start 147.355 82.805) (end 150 80.16) (width 0.75) (layer F.Cu) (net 7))
 (segment (start 99.3394 84.4042) (end 99.5958 84.4042) (width 0.75) (layer F.Cu) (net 7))
 (via (at 132.2 97.6) (size 0.8) (layers F.Cu B.Cu) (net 7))
 (segment (start 138.5 80.0984) (end 137.7 80.8984) (width 0.75) (layer B.Cu) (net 10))
 (segment (start 137.7 80.8984) (end 137.7 96.1) (width 0.75) (layer B.Cu) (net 10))
 (segment (start 137.7 96.1) (end 132.2 101.6) (width 0.75) (layer B.Cu) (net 10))
 (segment (start 132.2 101.6) (end 112.6 101.6) (width 0.75) (layer B.Cu) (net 10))
 (segment (start 129.438 71.3608) (end 129.438 69.0812) (width 0.75) (layer F.Cu) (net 13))
 (segment (start 129.438 69.0812) (end 133.96 64.56) (width 0.75) (layer F.Cu) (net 13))
 (segment (start 129.438 74.3616) (end 129.438 78.9808) (width 0.75) (layer B.Cu) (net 13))
 (segment (start 129.438 74.3616) (end 126.898 76.9016) (width 0.75) (layer B.Cu) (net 13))
 (segment (start 126.898 76.9016) (end 126.898 78.9808) (width 0.75) (layer B.Cu) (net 13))
 (segment (start 129.438 71.3608) (end 129.438 74.3616) (width 0.75) (layer B.Cu) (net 13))
 (segment (start 112.6 96.52) (end 115.72 96.52) (width 0.75) (layer B.Cu) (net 11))
 (segment (start 115.72 96.52) (end 119.75 100.55) (width 0.75) (layer B.Cu) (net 11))
 (segment (start 119.75 100.55) (end 131.765 100.55) (width 0.75) (layer B.Cu) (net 11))
 (segment (start 131.765 100.55) (end 131.765 100.435) (width 0.75) (layer B.Cu) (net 11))
 (segment (start 131.765 100.435) (end 135 97.2) (width 0.75) (layer B.Cu) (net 11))
 (segment (start 135 97.2) (end 135 94.36) (width 0.75) (layer B.Cu) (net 11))
 (segment (start 154 80) (end 150 84) (width 1) (layer B.Cu) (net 12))
 (segment (start 150 84) (end 150 96.6) (width 1) (layer B.Cu) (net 12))
 (segment (start 150 96.6) (end 147 99.6) (width 1) (layer B.Cu) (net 12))
 (segment (start 147 99.6) (end 145 99.6) (width 1) (layer B.Cu) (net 12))
 (segment (start 117.4 88) (end 117.4 96.8) (width 0.75) (layer F.Cu) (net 14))
 (segment (start 117.4 96.8) (end 115.14 99.06) (width 0.75) (layer F.Cu) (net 14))
 (segment (start 121.818 78.9808) (end 117.4 83.3992) (width 0.75) (layer B.Cu) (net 14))
 (segment (start 117.4 83.3992) (end 117.4 88) (width 0.75) (layer B.Cu) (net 14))
 (via (at 117.4 88) (size 0.8) (layers F.Cu B.Cu) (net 14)))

